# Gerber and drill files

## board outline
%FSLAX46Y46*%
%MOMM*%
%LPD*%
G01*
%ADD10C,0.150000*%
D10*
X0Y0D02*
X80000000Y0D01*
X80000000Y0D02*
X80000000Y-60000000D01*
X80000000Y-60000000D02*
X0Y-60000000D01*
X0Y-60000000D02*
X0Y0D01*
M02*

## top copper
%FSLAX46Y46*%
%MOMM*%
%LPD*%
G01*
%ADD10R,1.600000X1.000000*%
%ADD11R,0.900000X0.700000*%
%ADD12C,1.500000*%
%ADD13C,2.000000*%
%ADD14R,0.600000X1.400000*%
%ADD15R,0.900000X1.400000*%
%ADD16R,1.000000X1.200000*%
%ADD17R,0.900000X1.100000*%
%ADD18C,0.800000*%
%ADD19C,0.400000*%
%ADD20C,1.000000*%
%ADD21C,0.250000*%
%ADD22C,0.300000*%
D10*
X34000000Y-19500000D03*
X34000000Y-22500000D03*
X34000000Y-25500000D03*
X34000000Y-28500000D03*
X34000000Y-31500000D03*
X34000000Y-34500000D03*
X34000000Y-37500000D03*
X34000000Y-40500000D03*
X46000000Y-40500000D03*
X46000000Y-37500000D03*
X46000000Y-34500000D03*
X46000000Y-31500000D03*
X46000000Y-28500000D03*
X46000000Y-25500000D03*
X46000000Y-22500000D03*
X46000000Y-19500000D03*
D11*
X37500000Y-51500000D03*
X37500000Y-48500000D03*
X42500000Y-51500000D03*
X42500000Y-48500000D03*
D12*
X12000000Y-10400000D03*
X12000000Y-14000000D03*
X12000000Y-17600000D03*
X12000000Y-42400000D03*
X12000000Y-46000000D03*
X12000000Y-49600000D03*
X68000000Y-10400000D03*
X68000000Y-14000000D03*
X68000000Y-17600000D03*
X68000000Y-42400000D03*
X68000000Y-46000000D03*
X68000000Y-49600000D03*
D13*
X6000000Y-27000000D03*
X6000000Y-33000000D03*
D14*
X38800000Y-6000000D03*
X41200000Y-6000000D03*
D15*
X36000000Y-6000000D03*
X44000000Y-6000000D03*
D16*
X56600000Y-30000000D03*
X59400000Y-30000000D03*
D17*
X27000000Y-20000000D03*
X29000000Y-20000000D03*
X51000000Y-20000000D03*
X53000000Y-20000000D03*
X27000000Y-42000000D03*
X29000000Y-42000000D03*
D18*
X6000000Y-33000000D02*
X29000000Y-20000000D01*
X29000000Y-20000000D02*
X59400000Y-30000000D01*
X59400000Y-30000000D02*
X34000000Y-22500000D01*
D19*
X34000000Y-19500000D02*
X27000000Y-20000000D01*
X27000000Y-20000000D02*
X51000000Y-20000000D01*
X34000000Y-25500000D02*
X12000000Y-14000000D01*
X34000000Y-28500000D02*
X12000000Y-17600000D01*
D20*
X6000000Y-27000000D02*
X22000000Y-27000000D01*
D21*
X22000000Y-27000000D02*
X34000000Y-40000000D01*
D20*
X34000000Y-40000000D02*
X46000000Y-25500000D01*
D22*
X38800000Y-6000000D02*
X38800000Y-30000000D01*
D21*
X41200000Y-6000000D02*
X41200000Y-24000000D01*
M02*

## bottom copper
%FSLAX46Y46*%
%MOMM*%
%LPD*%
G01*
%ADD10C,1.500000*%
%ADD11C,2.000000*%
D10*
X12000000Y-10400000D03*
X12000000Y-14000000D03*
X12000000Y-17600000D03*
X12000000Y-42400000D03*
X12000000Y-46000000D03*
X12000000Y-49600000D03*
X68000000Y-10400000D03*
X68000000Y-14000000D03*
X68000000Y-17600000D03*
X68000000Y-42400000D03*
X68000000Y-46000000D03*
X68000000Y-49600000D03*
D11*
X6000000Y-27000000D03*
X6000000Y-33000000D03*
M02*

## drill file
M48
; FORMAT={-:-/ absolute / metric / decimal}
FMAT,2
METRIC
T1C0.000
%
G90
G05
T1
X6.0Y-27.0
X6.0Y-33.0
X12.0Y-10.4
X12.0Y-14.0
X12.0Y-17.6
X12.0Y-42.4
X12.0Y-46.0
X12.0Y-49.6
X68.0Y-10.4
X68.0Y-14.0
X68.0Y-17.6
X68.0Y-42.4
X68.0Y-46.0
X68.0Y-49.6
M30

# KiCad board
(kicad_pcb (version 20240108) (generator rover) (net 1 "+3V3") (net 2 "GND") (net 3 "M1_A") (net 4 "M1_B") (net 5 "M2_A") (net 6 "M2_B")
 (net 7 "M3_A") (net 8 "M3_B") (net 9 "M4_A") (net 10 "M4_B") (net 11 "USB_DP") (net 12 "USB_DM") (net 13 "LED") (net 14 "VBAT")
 (gr_line (start 0 0) (end 80.0 0) (layer "Edge.Cuts") (width 0.15))
 (gr_line (start 80.0 0) (end 80.0 60.0) (layer "Edge.Cuts") (width 0.15))
 (gr_line (start 80.0 60.0) (end 0 60.0) (layer "Edge.Cuts") (width 0.15))
 (gr_line (start 0 60.0) (end 0 0) (layer "Edge.Cuts") (width 0.15))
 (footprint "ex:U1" (at 40 30 0) (layer "F.Cu") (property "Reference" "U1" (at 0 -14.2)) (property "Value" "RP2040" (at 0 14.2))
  (pad "1" smd rect (at -6.0 -10.5) (size 1.6 1.0) (layers "F.Cu" "F.Mask") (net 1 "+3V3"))
  (pad "2" smd rect (at -6.0 -7.5) (size 1.6 1.0) (layers "F.Cu" "F.Mask") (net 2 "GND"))
  (pad "3" smd rect (at -6.0 -4.5) (size 1.6 1.0) (layers "F.Cu" "F.Mask") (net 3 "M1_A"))
  (pad "4" smd rect (at -6.0 -1.5) (size 1.6 1.0) (layers "F.Cu" "F.Mask") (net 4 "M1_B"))
  (pad "5" smd rect (at -6.0 1.5) (size 1.6 1.0) (layers "F.Cu" "F.Mask") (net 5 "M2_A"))
  (pad "6" smd rect (at -6.0 4.5) (size 1.6 1.0) (layers "F.Cu" "F.Mask") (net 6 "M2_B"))
  (pad "7" smd rect (at -6.0 7.5) (size 1.6 1.0) (layers "F.Cu" "F.Mask") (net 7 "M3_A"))
  (pad "8" smd rect (at -6.0 10.5) (size 1.6 1.0) (layers "F.Cu" "F.Mask") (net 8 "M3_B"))
  (pad "9" smd rect (at 6.0 10.5) (size 1.6 1.0) (layers "F.Cu" "F.Mask") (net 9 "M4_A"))
  (pad "10" smd rect (at 6.0 7.5) (size 1.6 1.0) (layers "F.Cu" "F.Mask") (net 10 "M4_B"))
  (pad "11" smd rect (at 6.0 4.5) (size 1.6 1.0) (layers "F.Cu" "F.Mask") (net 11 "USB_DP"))
  (pad "12" smd rect (at 6.0 1.5) (size 1.6 1.0) (layers "F.Cu" "F.Mask") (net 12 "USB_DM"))
  (pad "13" smd rect (at 6.0 -1.5) (size 1.6 1.0) (layers "F.Cu" "F.Mask") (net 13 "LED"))
  (pad "14" smd rect (at 6.0 -4.5) (size 1.6 1.0) (layers "F.Cu" "F.Mask") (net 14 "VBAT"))
  (pad "15" smd rect (at 6.0 -7.5) (size 1.6 1.0) (layers "F.Cu" "F.Mask") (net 2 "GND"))
  (pad "16" smd rect (at 6.0 -10.5) (size 1.6 1.0) (layers "F.Cu" "F.Mask") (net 1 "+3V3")))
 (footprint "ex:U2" (at 40 50 0) (layer "F.Cu") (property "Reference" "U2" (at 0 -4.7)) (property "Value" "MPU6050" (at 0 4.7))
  (pad "1" smd rect (at -2.5 1.5) (size 0.9 0.7) (layers "F.Cu" "F.Mask") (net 1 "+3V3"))
  (pad "2" smd rect (at -2.5 -1.5) (size 0.9 0.7) (layers "F.Cu" "F.Mask") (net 2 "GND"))
  (pad "3" smd rect (at 2.5 1.5) (size 0.9 0.7) (layers "F.Cu" "F.Mask") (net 11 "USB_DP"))
  (pad "4" smd rect (at 2.5 -1.5) (size 0.9 0.7) (layers "F.Cu" "F.Mask") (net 12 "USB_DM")))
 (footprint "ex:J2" (at 12 14 0) (layer "F.Cu") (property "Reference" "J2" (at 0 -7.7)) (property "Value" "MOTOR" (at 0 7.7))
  (pad "1" thru_hole circle (at 0.0 -3.6) (size 1.5 1.5) (layers "*.Cu" "*.Mask") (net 14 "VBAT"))
  (pad "2" thru_hole circle (at 0.0 0.0) (size 1.5 1.5) (layers "*.Cu" "*.Mask") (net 3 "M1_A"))
  (pad "3" thru_hole circle (at 0.0 3.6) (size 1.5 1.5) (layers "*.Cu" "*.Mask") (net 4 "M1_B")))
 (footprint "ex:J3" (at 12 46 0) (layer "F.Cu") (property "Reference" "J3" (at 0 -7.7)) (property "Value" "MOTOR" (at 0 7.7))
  (pad "1" thru_hole circle (at 0.0 -3.6) (size 1.5 1.5) (layers "*.Cu" "*.Mask") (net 14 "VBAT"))
  (pad "2" thru_hole circle (at 0.0 0.0) (size 1.5 1.5) (layers "*.Cu" "*.Mask") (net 5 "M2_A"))
  (pad "3" thru_hole circle (at 0.0 3.6) (size 1.5 1.5) (layers "*.Cu" "*.Mask") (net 6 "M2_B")))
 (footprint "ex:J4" (at 68 14 0) (layer "F.Cu") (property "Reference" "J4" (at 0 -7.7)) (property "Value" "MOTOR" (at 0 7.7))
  (pad "1" thru_hole circle (at 0.0 -3.6) (size 1.5 1.5) (layers "*.Cu" "*.Mask") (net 14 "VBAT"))
  (pad "2" thru_hole circle (at 0.0 0.0) (size 1.5 1.5) (layers "*.Cu" "*.Mask") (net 7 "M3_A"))
  (pad "3" thru_hole circle (at 0.0 3.6) (size 1.5 1.5) (layers "*.Cu" "*.Mask") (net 8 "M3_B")))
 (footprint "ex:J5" (at 68 46 0) (layer "F.Cu") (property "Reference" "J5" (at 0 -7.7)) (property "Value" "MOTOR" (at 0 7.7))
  (pad "1" thru_hole circle (at 0.0 -3.6) (size 1.5 1.5) (layers "*.Cu" "*.Mask") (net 14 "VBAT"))
  (pad "2" thru_hole circle (at 0.0 0.0) (size 1.5 1.5) (layers "*.Cu" "*.Mask") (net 9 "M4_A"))
  (pad "3" thru_hole circle (at 0.0 3.6) (size 1.5 1.5) (layers "*.Cu" "*.Mask") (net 10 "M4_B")))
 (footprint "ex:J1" (at 6 30 0) (layer "F.Cu") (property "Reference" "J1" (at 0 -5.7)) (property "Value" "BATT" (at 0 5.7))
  (pad "1" thru_hole circle (at 0 -3) (size 2.0 2.0) (layers "*.Cu" "*.Mask") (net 14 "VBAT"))
  (pad "2" thru_hole circle (at 0 3) (size 2.0 2.0) (layers "*.Cu" "*.Mask") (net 2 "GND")))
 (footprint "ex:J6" (at 40 6 0) (layer "F.Cu") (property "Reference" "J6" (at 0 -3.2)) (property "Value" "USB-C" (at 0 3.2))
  (pad "1" smd rect (at -1.2 0) (size 0.6 1.4) (layers "F.Cu" "F.Mask") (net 11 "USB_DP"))
  (pad "2" smd rect (at 1.2 0) (size 0.6 1.4) (layers "F.Cu" "F.Mask") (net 12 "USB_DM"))
  (pad "3" smd rect (at -4.0 0) (size 0.9 1.4) (layers "F.Cu" "F.Mask") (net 14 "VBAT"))
  (pad "4" smd rect (at 4.0 0) (size 0.9 1.4) (layers "F.Cu" "F.Mask") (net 2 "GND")))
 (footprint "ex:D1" (at 58 30 0) (layer "F.Cu") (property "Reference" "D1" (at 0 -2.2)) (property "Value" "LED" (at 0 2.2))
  (pad "1" smd rect (at -1.4 0) (size 1.0 1.2) (layers "F.Cu" "F.Mask") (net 13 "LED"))
  (pad "2" smd rect (at 1.4 0) (size 1.0 1.2) (layers "F.Cu" "F.Mask") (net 2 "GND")))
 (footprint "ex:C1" (at 28 20 0) (layer "F.Cu") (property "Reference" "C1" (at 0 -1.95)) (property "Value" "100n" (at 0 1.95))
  (pad "1" smd rect (at -1.0 0) (size 0.9 1.1) (layers "F.Cu" "F.Mask") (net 1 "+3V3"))
  (pad "2" smd rect (at 1.0 0) (size 0.9 1.1) (layers "F.Cu" "F.Mask") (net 2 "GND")))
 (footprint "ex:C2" (at 52 20 0) (layer "F.Cu") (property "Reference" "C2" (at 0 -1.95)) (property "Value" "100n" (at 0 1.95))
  (pad "1" smd rect (at -1.0 0) (size 0.9 1.1) (layers "F.Cu" "F.Mask") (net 1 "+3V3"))
  (pad "2" smd rect (at 1.0 0) (size 0.9 1.1) (layers "F.Cu" "F.Mask") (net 2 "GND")))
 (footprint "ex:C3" (at 28 42 0) (layer "F.Cu") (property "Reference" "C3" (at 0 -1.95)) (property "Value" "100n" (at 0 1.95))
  (pad "1" smd rect (at -1.0 0) (size 0.9 1.1) (layers "F.Cu" "F.Mask") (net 1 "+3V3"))
  (pad "2" smd rect (at 1.0 0) (size 0.9 1.1) (layers "F.Cu" "F.Mask") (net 2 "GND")))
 (segment (start 6.000 33.000) (end 29.000 20.000) (width 0.8) (layer "F.Cu") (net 2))
 (segment (start 29.000 20.000) (end 59.400 30.000) (width 0.8) (layer "F.Cu") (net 2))
 (segment (start 59.400 30.000) (end 34.000 22.500) (width 0.8) (layer "F.Cu") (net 2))
 (segment (start 34.000 19.500) (end 27.000 20.000) (width 0.4) (layer "F.Cu") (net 1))
 (segment (start 27.000 20.000) (end 51.000 20.000) (width 0.4) (layer "F.Cu") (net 1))
 (segment (start 34.000 25.500) (end 12.000 14.000) (width 0.4) (layer "F.Cu") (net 3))
 (segment (start 34.000 28.500) (end 12.000 17.600) (width 0.4) (layer "F.Cu") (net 4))
 (segment (start 6.000 27.000) (end 22.000 27.000) (width 1.0) (layer "F.Cu") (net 14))
 (segment (start 22.000 27.000) (end 34.000 40.000) (width 0.25) (layer "F.Cu") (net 14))
 (segment (start 34.000 40.000) (end 46.000 25.500) (width 1.0) (layer "F.Cu") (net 14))
 (segment (start 38.800 6.000) (end 38.800 30.000) (width 0.3) (layer "F.Cu") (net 12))
 (segment (start 41.200 6.000) (end 41.200 24.000) (width 0.25) (layer "F.Cu") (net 11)))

